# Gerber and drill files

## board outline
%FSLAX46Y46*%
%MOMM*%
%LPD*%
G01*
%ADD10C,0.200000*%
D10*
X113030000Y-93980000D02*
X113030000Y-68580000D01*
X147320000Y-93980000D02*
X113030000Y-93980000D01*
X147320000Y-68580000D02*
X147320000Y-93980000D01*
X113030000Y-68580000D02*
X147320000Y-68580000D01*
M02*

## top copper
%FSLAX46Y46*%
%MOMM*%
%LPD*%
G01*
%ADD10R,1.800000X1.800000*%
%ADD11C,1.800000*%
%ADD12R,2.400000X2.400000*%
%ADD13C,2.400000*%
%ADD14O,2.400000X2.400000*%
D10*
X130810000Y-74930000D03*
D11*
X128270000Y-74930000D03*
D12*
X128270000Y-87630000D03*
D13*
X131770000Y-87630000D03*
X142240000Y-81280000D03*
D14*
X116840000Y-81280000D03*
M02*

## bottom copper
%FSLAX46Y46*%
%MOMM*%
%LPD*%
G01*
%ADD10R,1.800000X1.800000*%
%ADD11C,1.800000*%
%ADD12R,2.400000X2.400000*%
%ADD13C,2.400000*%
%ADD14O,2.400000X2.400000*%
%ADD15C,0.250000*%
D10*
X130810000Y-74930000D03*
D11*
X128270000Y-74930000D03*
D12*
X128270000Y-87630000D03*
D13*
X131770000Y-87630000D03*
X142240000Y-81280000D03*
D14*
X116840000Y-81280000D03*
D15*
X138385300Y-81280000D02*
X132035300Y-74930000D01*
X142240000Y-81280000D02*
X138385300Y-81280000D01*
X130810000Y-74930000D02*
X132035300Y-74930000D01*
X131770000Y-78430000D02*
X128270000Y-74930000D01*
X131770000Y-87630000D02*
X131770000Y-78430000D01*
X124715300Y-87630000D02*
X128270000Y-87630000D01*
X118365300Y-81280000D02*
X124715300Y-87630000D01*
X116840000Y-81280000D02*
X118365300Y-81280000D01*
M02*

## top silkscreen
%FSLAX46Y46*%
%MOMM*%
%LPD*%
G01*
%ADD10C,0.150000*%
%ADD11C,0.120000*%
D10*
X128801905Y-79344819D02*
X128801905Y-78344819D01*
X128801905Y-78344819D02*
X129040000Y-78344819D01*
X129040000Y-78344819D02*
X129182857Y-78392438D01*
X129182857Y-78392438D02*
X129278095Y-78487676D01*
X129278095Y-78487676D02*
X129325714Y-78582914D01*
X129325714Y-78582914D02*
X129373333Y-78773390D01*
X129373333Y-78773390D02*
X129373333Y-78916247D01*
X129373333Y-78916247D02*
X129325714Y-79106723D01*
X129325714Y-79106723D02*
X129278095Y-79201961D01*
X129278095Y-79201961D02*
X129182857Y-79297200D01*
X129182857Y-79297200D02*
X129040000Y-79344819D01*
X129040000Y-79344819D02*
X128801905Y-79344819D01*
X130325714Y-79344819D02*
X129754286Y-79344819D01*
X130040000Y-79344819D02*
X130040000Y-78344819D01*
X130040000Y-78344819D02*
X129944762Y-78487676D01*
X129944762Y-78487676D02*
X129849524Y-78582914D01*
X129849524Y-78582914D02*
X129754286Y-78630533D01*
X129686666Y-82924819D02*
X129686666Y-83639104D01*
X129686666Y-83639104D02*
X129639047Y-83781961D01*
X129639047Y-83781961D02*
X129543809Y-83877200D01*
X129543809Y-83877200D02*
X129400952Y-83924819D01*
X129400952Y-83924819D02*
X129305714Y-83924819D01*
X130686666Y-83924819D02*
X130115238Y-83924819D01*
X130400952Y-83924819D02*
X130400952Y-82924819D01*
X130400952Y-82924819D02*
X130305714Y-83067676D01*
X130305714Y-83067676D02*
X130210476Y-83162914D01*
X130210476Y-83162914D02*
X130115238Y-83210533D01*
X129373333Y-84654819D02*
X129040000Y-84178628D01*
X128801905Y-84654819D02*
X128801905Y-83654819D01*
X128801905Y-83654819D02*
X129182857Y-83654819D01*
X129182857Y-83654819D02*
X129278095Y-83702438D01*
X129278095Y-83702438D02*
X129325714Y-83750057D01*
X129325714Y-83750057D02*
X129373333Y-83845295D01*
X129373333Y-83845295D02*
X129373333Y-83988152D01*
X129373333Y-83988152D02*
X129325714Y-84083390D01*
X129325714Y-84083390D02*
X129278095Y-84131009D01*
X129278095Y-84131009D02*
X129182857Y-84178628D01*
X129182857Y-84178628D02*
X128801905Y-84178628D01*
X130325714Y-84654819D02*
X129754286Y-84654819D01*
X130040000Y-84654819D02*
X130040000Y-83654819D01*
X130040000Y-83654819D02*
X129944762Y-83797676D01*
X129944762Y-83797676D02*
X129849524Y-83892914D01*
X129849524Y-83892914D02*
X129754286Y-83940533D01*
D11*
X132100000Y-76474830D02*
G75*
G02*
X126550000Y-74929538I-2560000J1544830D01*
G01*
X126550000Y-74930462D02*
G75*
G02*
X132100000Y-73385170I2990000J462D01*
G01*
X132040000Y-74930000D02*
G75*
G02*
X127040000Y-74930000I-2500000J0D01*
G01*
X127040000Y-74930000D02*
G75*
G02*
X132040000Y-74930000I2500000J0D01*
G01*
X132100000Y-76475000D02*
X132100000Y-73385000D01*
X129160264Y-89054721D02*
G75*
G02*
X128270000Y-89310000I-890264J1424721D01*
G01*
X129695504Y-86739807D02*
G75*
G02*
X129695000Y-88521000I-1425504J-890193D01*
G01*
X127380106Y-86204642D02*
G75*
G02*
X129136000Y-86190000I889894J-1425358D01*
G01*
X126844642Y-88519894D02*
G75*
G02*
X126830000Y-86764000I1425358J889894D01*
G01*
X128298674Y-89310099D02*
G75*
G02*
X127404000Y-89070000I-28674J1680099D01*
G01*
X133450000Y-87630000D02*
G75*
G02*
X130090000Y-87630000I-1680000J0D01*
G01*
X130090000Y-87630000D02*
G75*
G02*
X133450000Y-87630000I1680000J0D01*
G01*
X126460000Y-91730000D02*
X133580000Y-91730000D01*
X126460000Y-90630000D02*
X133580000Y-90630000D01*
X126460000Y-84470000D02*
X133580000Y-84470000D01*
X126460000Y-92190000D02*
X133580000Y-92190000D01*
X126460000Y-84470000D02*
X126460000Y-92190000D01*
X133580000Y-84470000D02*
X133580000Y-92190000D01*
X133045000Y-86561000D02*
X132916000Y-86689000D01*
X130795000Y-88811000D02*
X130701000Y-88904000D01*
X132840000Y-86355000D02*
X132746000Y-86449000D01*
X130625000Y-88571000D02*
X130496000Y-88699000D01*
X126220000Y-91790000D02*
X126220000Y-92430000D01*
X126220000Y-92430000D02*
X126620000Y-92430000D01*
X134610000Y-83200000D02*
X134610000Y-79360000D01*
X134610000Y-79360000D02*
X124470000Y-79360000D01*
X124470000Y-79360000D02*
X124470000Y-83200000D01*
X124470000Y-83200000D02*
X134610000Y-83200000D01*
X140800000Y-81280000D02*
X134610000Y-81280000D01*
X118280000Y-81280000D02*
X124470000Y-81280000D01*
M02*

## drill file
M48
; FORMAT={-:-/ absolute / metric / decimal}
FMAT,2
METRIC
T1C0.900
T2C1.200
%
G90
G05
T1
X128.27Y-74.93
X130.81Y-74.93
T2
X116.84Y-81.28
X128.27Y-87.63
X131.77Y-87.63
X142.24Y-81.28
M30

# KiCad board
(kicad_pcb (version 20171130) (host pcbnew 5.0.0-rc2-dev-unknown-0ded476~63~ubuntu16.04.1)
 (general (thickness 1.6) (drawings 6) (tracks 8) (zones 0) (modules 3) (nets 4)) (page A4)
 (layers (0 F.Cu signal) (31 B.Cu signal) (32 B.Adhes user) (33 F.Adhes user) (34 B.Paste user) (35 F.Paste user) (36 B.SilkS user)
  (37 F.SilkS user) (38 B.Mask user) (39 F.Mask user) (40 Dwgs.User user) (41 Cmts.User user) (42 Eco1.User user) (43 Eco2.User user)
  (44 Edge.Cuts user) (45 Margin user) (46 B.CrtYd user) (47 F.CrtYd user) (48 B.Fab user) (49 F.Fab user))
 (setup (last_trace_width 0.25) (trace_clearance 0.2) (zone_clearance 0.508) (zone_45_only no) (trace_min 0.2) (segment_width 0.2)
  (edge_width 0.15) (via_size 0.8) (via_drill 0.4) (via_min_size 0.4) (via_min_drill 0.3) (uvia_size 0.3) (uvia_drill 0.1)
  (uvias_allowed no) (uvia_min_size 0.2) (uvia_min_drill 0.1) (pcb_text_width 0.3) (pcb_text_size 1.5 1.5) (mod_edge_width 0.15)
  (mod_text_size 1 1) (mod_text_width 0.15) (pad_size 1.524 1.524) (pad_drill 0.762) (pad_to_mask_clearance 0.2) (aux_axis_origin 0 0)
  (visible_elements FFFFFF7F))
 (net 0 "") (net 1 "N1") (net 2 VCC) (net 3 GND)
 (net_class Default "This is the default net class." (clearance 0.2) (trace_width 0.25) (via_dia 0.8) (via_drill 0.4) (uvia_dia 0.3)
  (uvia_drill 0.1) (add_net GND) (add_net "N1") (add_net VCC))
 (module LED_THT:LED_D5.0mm (layer F.Cu) (at 130.81 74.93 180)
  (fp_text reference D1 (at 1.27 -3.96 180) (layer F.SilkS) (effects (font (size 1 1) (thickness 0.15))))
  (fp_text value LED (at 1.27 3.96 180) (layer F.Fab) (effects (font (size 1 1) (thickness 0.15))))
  (fp_arc (start 1.27 0) (end -1.29 -1.54483) (angle 148.9) (layer F.SilkS) (width 0.12))
  (fp_arc (start 1.27 0) (end -1.29 1.54483) (angle -148.9) (layer F.SilkS) (width 0.12))
  (fp_circle (center 1.27 0) (end 3.77 0) (layer F.SilkS) (width 0.12))
  (fp_line (start -1.29 -1.545) (end -1.29 1.545) (layer F.SilkS) (width 0.12))
  (pad 1 thru_hole rect (at 0 0 180) (size 1.8 1.8) (drill 0.9) (layers *.Cu *.Mask) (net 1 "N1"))
  (pad 2 thru_hole circle (at 2.54 0 180) (size 1.8 1.8) (drill 0.9) (layers *.Cu *.Mask) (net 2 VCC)))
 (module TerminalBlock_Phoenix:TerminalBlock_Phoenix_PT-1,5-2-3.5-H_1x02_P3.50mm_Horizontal (layer F.Cu) (at 128.27 87.63)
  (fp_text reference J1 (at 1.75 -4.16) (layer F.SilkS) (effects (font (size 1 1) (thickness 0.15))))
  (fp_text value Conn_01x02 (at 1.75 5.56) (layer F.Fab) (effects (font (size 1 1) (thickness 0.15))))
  (fp_arc (start 0 0) (end 0 1.68) (angle -32) (layer F.SilkS) (width 0.12))
  (fp_arc (start 0 0) (end 1.425 0.891) (angle -64) (layer F.SilkS) (width 0.12))
  (fp_arc (start 0 0) (end 0.866 -1.44) (angle -63) (layer F.SilkS) (width 0.12))
  (fp_arc (start 0 0) (end -1.44 -0.866) (angle -63) (layer F.SilkS) (width 0.12))
  (fp_arc (start 0 0) (end -0.866 1.44) (angle -32) (layer F.SilkS) (width 0.12))
  (fp_circle (center 3.5 0) (end 5.18 0) (layer F.SilkS) (width 0.12))
  (fp_line (start -1.81 4.1) (end 5.31 4.1) (layer F.SilkS) (width 0.12))
  (fp_line (start -1.81 3) (end 5.31 3) (layer F.SilkS) (width 0.12))
  (fp_line (start -1.81 -3.16) (end 5.31 -3.16) (layer F.SilkS) (width 0.12))
  (fp_line (start -1.81 4.56) (end 5.31 4.56) (layer F.SilkS) (width 0.12))
  (fp_line (start -1.81 -3.16) (end -1.81 4.56) (layer F.SilkS) (width 0.12))
  (fp_line (start 5.31 -3.16) (end 5.31 4.56) (layer F.SilkS) (width 0.12))
  (fp_line (start 4.775 -1.069) (end 4.646 -0.941) (layer F.SilkS) (width 0.12))
  (fp_line (start 2.525 1.181) (end 2.431 1.274) (layer F.SilkS) (width 0.12))
  (fp_line (start 4.57 -1.275) (end 4.476 -1.181) (layer F.SilkS) (width 0.12))
  (fp_line (start 2.355 0.941) (end 2.226 1.069) (layer F.SilkS) (width 0.12))
  (fp_line (start -2.05 4.16) (end -2.05 4.8) (layer F.SilkS) (width 0.12))
  (fp_line (start -2.05 4.8) (end -1.65 4.8) (layer F.SilkS) (width 0.12))
  (pad 1 thru_hole rect (at 0 0) (size 2.4 2.4) (drill 1.2) (layers *.Cu *.Mask) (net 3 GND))
  (pad 2 thru_hole circle (at 3.5 0) (size 2.4 2.4) (drill 1.2) (layers *.Cu *.Mask) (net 2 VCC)))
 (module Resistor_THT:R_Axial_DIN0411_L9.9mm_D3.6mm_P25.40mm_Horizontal (layer F.Cu) (at 142.24 81.28 180)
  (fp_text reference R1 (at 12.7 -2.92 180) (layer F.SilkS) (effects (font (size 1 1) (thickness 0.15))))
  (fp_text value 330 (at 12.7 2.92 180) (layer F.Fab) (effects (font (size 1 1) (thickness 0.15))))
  (fp_line (start 7.63 -1.92) (end 7.63 1.92) (layer F.SilkS) (width 0.12))
  (fp_line (start 7.63 1.92) (end 17.77 1.92) (layer F.SilkS) (width 0.12))
  (fp_line (start 17.77 1.92) (end 17.77 -1.92) (layer F.SilkS) (width 0.12))
  (fp_line (start 17.77 -1.92) (end 7.63 -1.92) (layer F.SilkS) (width 0.12))
  (fp_line (start 1.44 0) (end 7.63 0) (layer F.SilkS) (width 0.12))
  (fp_line (start 23.96 0) (end 17.77 0) (layer F.SilkS) (width 0.12))
  (pad 1 thru_hole circle (at 0 0 180) (size 2.4 2.4) (drill 1.2) (layers *.Cu *.Mask) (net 1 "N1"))
  (pad 2 thru_hole oval (at 25.4 0 180) (size 2.4 2.4) (drill 1.2) (layers *.Cu *.Mask) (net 3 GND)))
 (gr_line (start 113.03 93.98) (end 113.03 68.58) (layer Edge.Cuts) (width 0.2))
 (gr_line (start 147.32 93.98) (end 113.03 93.98) (layer Edge.Cuts) (width 0.2))
 (gr_line (start 147.32 68.58) (end 147.32 93.98) (layer Edge.Cuts) (width 0.2))
 (gr_line (start 113.03 68.58) (end 147.32 68.58) (layer Edge.Cuts) (width 0.2))
 (segment (start 138.3853 81.28) (end 132.0353 74.93) (width 0.25) (layer B.Cu) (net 1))
 (segment (start 142.24 81.28) (end 138.3853 81.28) (width 0.25) (layer B.Cu) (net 1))
 (segment (start 130.81 74.93) (end 132.0353 74.93) (width 0.25) (layer B.Cu) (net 1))
 (segment (start 131.77 78.43) (end 128.27 74.93) (width 0.25) (layer B.Cu) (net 2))
 (segment (start 131.77 87.63) (end 131.77 78.43) (width 0.25) (layer B.Cu) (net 2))
 (segment (start 124.7153 87.63) (end 128.27 87.63) (width 0.25) (layer B.Cu) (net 3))
 (segment (start 118.3653 81.28) (end 124.7153 87.63) (width 0.25) (layer B.Cu) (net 3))
 (segment (start 116.84 81.28) (end 118.3653 81.28) (width 0.25) (layer B.Cu) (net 3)))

